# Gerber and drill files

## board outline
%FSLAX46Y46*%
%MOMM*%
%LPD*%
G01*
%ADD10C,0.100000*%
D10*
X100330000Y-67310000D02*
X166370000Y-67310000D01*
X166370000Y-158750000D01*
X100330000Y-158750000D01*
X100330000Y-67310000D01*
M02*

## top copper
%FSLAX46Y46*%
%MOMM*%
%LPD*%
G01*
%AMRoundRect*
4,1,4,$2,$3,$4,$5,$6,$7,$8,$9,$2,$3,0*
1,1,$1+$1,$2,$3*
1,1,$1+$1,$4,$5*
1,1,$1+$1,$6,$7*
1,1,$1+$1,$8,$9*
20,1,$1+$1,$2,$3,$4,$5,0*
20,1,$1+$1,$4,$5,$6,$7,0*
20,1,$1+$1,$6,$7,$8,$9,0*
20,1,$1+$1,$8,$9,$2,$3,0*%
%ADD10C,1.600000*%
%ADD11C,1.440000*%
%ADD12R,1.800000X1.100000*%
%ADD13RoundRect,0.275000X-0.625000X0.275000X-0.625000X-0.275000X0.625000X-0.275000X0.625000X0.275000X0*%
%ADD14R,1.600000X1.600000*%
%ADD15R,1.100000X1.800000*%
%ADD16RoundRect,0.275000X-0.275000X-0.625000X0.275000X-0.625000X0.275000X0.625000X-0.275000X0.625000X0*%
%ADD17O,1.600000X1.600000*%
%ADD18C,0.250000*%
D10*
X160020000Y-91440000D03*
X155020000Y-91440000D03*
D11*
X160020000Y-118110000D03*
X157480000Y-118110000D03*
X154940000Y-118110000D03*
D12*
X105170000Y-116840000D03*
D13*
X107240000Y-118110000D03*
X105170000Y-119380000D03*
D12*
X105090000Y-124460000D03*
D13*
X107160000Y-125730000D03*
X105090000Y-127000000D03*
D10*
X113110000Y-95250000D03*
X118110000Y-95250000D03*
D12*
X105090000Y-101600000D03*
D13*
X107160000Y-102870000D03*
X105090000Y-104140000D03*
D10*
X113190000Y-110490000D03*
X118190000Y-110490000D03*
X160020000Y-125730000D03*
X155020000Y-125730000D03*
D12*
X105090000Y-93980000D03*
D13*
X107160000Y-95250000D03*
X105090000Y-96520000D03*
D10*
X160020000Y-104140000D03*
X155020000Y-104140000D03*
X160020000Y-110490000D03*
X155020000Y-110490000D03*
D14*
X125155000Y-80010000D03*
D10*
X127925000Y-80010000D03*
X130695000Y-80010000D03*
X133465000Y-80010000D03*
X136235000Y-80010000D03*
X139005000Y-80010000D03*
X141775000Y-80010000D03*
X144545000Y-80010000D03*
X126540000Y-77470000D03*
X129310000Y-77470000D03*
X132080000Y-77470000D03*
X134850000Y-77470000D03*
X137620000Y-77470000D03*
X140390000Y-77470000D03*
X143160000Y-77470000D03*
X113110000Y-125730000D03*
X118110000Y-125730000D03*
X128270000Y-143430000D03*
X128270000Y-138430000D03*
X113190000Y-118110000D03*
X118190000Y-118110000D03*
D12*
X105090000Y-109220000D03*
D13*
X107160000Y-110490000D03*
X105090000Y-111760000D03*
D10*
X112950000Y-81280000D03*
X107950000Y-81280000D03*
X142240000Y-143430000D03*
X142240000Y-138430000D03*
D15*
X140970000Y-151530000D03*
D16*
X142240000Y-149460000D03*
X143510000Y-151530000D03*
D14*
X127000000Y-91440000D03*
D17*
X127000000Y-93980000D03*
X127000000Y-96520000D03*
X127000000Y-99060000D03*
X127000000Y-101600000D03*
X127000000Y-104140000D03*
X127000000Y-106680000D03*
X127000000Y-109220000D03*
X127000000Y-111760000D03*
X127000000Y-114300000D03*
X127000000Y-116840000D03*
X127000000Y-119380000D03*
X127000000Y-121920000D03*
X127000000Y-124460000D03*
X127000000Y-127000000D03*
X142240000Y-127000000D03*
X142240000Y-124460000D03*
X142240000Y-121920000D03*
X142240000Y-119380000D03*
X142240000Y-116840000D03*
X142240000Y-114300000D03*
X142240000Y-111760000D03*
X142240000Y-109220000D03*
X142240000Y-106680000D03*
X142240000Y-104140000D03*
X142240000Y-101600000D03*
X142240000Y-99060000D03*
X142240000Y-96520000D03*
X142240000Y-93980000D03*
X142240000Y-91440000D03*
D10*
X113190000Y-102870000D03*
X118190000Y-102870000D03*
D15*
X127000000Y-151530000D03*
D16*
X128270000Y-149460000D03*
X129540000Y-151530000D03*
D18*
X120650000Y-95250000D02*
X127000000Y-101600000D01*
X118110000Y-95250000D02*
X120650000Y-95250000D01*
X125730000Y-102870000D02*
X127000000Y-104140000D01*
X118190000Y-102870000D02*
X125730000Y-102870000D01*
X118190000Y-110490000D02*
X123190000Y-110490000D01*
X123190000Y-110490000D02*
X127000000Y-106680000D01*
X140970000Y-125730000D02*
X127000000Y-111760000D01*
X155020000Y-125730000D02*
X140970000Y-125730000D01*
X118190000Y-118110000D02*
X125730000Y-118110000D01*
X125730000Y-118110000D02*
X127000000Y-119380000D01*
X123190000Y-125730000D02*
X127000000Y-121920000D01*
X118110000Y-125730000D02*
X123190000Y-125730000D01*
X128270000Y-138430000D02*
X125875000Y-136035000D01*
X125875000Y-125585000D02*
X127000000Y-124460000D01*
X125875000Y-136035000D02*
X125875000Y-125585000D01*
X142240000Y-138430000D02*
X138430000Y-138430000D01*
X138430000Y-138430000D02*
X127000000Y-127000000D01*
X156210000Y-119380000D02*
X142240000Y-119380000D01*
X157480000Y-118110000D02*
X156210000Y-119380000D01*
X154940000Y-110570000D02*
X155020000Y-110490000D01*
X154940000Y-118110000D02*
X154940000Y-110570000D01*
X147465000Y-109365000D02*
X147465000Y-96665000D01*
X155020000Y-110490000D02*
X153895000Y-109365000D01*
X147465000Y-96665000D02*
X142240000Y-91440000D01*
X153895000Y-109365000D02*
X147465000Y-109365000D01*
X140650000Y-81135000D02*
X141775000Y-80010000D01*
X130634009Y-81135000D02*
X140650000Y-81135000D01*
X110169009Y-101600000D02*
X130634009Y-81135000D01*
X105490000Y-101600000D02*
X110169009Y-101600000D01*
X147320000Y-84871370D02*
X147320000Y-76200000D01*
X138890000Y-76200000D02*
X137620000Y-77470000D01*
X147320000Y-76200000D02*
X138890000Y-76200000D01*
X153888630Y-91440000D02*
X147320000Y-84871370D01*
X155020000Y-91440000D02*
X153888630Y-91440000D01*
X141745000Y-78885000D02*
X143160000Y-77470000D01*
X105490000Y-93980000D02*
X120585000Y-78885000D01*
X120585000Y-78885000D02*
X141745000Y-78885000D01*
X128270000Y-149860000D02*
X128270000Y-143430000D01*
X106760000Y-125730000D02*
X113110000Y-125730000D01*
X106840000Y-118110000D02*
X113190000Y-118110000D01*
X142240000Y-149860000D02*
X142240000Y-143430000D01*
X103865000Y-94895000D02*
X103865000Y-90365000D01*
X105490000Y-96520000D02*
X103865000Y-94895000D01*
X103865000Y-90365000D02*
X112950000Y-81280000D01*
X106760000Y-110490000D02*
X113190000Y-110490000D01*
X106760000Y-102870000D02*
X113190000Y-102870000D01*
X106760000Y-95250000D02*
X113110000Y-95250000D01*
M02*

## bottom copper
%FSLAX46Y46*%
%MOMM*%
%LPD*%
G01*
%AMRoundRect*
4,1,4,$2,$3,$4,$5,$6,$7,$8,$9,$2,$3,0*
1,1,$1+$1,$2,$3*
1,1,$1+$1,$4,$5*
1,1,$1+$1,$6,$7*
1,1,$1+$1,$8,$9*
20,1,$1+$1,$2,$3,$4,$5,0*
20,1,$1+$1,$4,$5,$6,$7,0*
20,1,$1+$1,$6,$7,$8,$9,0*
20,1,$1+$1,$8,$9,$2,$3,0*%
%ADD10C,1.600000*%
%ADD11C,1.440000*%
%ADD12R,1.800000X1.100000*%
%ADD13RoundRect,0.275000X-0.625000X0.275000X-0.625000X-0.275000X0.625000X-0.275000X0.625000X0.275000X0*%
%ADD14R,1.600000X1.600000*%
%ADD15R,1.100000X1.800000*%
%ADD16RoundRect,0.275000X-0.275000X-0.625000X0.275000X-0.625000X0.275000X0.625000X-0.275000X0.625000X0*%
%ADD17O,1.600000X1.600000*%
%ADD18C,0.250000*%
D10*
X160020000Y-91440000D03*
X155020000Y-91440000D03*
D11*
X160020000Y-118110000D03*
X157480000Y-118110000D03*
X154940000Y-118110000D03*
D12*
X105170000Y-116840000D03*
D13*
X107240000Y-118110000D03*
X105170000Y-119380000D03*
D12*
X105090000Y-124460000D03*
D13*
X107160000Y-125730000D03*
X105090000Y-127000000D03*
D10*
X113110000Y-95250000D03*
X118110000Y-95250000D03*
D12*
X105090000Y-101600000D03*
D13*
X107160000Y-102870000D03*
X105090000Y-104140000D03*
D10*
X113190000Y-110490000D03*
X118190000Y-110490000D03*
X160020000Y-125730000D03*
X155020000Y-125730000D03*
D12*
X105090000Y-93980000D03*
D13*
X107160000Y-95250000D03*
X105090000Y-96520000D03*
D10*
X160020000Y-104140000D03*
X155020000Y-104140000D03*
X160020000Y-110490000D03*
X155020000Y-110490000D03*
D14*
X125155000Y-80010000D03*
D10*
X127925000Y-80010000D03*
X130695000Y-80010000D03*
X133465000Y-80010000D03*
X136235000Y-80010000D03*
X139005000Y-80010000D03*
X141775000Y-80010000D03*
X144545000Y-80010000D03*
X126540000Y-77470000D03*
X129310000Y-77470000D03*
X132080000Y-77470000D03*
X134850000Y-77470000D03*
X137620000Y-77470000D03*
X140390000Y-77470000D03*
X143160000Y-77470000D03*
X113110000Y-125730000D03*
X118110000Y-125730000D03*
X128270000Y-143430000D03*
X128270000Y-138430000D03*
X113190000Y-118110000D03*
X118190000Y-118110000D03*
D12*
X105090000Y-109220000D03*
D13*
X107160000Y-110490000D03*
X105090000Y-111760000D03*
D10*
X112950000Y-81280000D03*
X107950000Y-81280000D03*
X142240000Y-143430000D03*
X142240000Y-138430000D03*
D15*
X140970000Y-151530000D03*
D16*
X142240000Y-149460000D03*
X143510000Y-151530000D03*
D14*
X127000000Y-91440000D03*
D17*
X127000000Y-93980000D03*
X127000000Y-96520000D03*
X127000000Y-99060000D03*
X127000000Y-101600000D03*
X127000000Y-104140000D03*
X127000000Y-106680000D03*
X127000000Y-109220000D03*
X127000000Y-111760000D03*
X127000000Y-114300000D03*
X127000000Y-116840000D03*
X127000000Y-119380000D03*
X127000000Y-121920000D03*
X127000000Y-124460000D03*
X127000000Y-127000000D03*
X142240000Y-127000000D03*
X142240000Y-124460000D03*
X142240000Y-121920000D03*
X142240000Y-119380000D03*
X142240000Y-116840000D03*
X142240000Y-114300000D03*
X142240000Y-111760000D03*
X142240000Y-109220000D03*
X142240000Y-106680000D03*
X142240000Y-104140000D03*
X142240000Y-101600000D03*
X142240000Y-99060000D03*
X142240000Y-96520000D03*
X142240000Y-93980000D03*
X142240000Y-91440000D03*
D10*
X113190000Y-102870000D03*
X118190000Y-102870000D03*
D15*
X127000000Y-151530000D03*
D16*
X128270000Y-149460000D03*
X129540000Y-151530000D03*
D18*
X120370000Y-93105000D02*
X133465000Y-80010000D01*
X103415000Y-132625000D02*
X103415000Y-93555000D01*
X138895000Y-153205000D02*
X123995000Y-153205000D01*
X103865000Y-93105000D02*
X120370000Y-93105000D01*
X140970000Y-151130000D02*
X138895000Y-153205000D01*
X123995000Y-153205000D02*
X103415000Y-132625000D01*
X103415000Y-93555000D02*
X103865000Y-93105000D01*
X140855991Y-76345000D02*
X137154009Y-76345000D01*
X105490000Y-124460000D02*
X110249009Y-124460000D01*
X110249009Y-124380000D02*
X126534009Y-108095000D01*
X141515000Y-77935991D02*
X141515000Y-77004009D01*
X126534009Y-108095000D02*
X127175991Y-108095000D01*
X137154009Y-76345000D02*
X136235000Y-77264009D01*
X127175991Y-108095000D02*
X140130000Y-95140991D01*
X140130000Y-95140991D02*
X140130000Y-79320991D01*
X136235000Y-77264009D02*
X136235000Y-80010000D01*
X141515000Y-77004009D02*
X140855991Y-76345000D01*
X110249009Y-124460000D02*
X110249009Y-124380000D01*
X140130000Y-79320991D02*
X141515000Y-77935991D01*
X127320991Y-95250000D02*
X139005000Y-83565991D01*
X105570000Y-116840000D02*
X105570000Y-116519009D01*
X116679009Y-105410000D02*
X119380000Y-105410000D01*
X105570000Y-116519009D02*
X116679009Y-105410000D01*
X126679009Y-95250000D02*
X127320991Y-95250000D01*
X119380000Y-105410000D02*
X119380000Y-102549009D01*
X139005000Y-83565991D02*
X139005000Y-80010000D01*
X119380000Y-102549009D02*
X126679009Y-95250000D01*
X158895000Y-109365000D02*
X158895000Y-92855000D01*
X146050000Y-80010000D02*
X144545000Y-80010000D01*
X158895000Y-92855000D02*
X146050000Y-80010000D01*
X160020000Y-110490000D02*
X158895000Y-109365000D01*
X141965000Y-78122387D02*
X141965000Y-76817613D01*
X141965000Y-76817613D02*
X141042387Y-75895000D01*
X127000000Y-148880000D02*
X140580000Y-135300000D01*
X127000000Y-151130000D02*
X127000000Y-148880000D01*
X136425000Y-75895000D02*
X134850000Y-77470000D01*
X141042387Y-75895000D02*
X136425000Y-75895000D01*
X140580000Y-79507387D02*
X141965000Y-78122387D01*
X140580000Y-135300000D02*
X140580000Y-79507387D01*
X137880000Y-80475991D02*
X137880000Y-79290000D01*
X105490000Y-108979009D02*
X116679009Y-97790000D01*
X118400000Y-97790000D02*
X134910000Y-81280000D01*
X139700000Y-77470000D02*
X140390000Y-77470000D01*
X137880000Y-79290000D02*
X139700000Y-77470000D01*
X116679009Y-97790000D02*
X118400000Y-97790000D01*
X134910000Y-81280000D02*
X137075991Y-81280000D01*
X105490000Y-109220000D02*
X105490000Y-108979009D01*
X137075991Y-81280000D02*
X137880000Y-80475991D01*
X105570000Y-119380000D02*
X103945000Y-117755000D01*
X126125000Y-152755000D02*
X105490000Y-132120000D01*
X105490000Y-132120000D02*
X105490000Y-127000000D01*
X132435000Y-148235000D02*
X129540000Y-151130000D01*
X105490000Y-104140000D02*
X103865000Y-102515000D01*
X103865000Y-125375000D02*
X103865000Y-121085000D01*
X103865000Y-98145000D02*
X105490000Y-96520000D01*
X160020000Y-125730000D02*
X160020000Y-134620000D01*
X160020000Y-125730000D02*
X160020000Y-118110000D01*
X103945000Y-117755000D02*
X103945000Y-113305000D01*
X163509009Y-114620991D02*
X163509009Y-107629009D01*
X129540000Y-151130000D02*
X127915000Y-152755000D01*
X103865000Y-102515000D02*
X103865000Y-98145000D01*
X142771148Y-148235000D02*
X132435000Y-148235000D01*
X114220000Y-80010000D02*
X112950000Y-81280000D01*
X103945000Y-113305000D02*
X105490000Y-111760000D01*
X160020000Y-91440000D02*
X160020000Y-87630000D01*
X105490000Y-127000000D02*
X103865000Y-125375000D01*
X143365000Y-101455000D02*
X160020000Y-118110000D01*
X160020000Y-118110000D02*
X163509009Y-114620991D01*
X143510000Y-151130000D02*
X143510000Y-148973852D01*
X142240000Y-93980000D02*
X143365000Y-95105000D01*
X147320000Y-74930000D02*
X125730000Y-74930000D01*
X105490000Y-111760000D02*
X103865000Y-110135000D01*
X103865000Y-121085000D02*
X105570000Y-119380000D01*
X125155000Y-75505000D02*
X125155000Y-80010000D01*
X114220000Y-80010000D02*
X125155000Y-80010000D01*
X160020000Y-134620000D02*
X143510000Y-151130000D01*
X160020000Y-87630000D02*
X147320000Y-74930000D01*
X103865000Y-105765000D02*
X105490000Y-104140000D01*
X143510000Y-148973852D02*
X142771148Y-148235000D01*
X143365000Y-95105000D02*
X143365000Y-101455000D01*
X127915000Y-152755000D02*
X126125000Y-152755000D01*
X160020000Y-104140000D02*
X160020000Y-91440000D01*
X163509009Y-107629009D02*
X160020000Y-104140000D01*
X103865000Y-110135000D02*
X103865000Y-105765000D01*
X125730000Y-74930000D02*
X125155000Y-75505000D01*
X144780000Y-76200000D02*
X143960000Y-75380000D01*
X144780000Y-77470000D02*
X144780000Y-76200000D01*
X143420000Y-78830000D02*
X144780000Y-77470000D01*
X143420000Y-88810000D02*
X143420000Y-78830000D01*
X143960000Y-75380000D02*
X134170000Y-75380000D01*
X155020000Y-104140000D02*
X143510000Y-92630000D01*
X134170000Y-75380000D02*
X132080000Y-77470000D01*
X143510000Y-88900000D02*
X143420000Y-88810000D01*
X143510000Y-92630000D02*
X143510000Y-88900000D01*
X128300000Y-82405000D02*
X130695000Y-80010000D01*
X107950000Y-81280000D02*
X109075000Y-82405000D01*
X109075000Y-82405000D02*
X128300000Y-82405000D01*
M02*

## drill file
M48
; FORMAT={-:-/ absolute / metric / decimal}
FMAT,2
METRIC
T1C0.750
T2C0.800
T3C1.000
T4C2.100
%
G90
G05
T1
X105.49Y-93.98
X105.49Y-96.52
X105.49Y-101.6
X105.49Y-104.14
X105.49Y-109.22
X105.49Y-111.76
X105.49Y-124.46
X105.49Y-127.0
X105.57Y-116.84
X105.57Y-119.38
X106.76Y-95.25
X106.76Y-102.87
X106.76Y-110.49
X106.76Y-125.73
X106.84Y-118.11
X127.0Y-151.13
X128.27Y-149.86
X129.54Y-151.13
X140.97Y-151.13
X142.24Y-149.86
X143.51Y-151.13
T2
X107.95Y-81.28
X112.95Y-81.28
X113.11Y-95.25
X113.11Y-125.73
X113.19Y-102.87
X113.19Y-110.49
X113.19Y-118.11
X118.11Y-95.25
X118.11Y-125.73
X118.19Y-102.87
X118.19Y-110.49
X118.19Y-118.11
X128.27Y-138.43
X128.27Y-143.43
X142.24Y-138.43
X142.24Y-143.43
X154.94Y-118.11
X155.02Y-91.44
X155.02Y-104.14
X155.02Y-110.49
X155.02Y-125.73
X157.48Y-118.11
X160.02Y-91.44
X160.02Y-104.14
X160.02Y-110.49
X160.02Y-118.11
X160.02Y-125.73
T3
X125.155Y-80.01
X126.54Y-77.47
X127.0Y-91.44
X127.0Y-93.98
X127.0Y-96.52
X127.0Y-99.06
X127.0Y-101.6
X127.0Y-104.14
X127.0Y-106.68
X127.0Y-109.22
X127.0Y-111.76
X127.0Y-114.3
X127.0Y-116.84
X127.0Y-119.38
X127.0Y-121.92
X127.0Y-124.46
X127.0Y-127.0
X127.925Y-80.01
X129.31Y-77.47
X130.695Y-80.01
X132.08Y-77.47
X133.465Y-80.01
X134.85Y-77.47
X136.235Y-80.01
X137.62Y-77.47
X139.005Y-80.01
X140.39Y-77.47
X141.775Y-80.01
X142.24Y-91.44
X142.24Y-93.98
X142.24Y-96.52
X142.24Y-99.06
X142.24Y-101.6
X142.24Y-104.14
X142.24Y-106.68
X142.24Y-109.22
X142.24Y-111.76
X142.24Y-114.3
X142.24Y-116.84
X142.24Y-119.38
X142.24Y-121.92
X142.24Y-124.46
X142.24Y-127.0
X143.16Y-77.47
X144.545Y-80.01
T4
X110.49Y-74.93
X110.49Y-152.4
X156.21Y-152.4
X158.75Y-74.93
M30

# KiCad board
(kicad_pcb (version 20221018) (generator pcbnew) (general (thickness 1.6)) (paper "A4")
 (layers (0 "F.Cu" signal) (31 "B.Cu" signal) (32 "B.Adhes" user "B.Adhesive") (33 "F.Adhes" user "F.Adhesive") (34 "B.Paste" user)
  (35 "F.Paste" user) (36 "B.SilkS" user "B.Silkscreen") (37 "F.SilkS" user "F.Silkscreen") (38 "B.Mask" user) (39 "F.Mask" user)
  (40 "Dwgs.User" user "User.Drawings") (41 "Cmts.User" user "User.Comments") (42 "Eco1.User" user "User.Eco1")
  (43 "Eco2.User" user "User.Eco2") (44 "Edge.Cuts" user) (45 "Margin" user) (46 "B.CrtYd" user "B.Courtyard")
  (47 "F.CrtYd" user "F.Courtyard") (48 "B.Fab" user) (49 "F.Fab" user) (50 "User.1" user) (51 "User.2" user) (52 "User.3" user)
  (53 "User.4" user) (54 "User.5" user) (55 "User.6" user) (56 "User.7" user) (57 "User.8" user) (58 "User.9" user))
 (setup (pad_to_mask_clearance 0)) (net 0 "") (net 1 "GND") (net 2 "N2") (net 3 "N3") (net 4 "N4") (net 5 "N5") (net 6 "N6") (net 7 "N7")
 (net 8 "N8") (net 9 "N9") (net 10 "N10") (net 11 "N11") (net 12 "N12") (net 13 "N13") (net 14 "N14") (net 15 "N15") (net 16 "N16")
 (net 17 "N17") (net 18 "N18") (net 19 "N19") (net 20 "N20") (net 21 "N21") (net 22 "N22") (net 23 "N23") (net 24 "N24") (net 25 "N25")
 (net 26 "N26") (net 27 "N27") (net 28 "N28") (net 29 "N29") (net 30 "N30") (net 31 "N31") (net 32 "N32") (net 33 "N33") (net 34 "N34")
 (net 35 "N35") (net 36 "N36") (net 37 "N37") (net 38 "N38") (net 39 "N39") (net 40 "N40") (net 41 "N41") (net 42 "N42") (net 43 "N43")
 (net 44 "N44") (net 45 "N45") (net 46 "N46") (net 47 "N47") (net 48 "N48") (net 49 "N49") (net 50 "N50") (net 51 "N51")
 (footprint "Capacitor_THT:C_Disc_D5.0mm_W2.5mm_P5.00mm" (layer "F.Cu") (at 160.02 91.44 180)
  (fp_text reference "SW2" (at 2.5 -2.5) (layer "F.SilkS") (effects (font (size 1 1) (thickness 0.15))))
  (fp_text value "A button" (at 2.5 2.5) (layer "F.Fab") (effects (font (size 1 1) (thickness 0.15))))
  (pad "1" thru_hole circle (at 0 0 180) (size 1.6 1.6) (drill 0.8) (layers "*.Cu" "*.Mask") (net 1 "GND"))
  (pad "2" thru_hole circle (at 5 0 180) (size 1.6 1.6) (drill 0.8) (layers "*.Cu" "*.Mask") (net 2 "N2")))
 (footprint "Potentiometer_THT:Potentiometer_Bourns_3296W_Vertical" (layer "F.Cu") (at 160.02 118.11)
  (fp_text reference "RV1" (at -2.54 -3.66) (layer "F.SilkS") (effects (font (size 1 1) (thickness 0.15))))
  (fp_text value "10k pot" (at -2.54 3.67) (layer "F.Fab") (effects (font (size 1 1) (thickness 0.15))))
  (pad "1" thru_hole circle (at 0 0) (size 1.44 1.44) (drill 0.8) (layers "*.Cu" "*.Mask") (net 1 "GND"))
  (pad "2" thru_hole circle (at -2.54 0) (size 1.44 1.44) (drill 0.8) (layers "*.Cu" "*.Mask") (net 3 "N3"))
  (pad "3" thru_hole circle (at -5.08 0) (size 1.44 1.44) (drill 0.8) (layers "*.Cu" "*.Mask") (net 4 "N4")))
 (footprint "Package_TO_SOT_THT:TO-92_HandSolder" (layer "F.Cu") (at 105.57 116.84 -90)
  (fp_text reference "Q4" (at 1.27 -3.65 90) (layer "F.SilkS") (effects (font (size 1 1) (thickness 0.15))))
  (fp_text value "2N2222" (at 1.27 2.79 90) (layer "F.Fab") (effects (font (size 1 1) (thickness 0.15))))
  (pad "1" thru_hole rect (at 0 0 270) (size 1.1 1.8) (drill 0.75 (offset 0 0.4)) (layers "*.Cu" "*.Mask") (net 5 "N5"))
  (pad "2" thru_hole roundrect (at 1.27 -1.27 270) (size 1.1 1.8) (drill 0.75 (offset 0 -0.4)) (layers "*.Cu" "*.Mask")
   (roundrect_rratio 0.25) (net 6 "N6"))
  (pad "3" thru_hole roundrect (at 2.54 0 270) (size 1.1 1.8) (drill 0.75 (offset 0 0.4)) (layers "*.Cu" "*.Mask") (roundrect_rratio 0.25)
   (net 1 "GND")))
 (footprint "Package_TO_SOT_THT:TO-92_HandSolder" (layer "F.Cu") (at 105.49 124.46 -90)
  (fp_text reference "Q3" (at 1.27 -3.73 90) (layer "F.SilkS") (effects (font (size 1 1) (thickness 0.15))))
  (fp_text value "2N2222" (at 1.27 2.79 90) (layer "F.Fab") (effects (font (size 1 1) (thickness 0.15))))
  (pad "1" thru_hole rect (at 0 0 270) (size 1.1 1.8) (drill 0.75 (offset 0 0.4)) (layers "*.Cu" "*.Mask") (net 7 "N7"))
  (pad "2" thru_hole roundrect (at 1.27 -1.27 270) (size 1.1 1.8) (drill 0.75 (offset 0 -0.4)) (layers "*.Cu" "*.Mask")
   (roundrect_rratio 0.25) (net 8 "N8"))
  (pad "3" thru_hole roundrect (at 2.54 0 270) (size 1.1 1.8) (drill 0.75 (offset 0 0.4)) (layers "*.Cu" "*.Mask") (roundrect_rratio 0.25)
   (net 1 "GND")))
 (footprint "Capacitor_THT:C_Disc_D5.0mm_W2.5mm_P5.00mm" (layer "F.Cu") (at 113.11 95.25)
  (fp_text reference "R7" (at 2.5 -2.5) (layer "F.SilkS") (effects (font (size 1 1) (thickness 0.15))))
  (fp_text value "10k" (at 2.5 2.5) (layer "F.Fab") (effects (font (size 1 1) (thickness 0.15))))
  (pad "1" thru_hole circle (at 0 0) (size 1.6 1.6) (drill 0.8) (layers "*.Cu" "*.Mask") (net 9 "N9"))
  (pad "2" thru_hole circle (at 5 0) (size 1.6 1.6) (drill 0.8) (layers "*.Cu" "*.Mask") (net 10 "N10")))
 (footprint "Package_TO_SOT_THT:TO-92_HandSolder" (layer "F.Cu") (at 105.49 101.6 -90)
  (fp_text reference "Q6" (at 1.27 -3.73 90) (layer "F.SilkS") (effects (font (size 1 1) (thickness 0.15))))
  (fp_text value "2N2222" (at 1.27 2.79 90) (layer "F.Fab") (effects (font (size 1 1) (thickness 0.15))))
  (pad "1" thru_hole rect (at 0 0 270) (size 1.1 1.8) (drill 0.75 (offset 0 0.4)) (layers "*.Cu" "*.Mask") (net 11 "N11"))
  (pad "2" thru_hole roundrect (at 1.27 -1.27 270) (size 1.1 1.8) (drill 0.75 (offset 0 -0.4)) (layers "*.Cu" "*.Mask")
   (roundrect_rratio 0.25) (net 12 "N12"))
  (pad "3" thru_hole roundrect (at 2.54 0 270) (size 1.1 1.8) (drill 0.75 (offset 0 0.4)) (layers "*.Cu" "*.Mask") (roundrect_rratio 0.25)
   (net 1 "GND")))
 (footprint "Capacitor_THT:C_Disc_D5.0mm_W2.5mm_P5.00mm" (layer "F.Cu") (at 113.19 110.49)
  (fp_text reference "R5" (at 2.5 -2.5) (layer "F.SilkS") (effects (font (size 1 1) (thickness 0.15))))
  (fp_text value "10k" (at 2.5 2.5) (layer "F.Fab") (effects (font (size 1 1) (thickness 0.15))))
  (pad "1" thru_hole circle (at 0 0) (size 1.6 1.6) (drill 0.8) (layers "*.Cu" "*.Mask") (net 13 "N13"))
  (pad "2" thru_hole circle (at 5 0) (size 1.6 1.6) (drill 0.8) (layers "*.Cu" "*.Mask") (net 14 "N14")))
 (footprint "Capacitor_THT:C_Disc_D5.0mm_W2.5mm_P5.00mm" (layer "F.Cu") (at 160.02 125.73 180)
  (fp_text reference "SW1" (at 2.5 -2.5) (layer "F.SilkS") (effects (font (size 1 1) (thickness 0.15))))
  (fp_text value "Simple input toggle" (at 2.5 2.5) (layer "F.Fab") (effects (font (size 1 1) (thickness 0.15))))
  (pad "1" thru_hole circle (at 0 0 180) (size 1.6 1.6) (drill 0.8) (layers "*.Cu" "*.Mask") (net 1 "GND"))
  (pad "2" thru_hole circle (at 5 0 180) (size 1.6 1.6) (drill 0.8) (layers "*.Cu" "*.Mask") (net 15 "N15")))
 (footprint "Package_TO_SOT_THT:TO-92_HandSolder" (layer "F.Cu") (at 105.49 93.98 -90)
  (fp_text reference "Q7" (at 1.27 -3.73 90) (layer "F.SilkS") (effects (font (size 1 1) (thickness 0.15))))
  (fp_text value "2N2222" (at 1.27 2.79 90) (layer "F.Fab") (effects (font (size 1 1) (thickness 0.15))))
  (pad "1" thru_hole rect (at 0 0 270) (size 1.1 1.8) (drill 0.75 (offset 0 0.4)) (layers "*.Cu" "*.Mask") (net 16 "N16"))
  (pad "2" thru_hole roundrect (at 1.27 -1.27 270) (size 1.1 1.8) (drill 0.75 (offset 0 -0.4)) (layers "*.Cu" "*.Mask")
   (roundrect_rratio 0.25) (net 9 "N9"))
  (pad "3" thru_hole roundrect (at 2.54 0 270) (size 1.1 1.8) (drill 0.75 (offset 0 0.4)) (layers "*.Cu" "*.Mask") (roundrect_rratio 0.25)
   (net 1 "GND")))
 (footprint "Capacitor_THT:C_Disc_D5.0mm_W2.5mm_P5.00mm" (layer "F.Cu") (at 160.02 104.14 180)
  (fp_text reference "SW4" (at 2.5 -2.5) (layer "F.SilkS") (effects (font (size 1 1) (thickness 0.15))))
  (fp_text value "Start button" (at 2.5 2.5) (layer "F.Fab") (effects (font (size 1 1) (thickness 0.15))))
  (pad "1" thru_hole circle (at 0 0 180) (size 1.6 1.6) (drill 0.8) (layers "*.Cu" "*.Mask") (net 1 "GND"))
  (pad "2" thru_hole circle (at 5 0 180) (size 1.6 1.6) (drill 0.8) (layers "*.Cu" "*.Mask") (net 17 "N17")))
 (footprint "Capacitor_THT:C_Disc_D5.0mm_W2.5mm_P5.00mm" (layer "F.Cu") (at 160.02 110.49 180)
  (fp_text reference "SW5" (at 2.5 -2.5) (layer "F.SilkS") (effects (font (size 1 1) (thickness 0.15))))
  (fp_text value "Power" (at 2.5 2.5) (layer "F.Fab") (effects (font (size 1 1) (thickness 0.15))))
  (pad "1" thru_hole circle (at 0 0 180) (size 1.6 1.6) (drill 0.8) (layers "*.Cu" "*.Mask") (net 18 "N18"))
  (pad "2" thru_hole circle (at 5 0 180) (size 1.6 1.6) (drill 0.8) (layers "*.Cu" "*.Mask") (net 4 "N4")))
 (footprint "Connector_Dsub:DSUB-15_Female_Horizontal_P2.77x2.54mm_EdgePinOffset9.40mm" (layer "F.Cu") (at 125.155 80.01 180)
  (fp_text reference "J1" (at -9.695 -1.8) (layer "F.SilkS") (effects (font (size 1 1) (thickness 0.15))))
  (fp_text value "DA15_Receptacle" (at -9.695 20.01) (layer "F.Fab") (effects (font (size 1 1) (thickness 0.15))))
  (pad "1" thru_hole rect (at 0 0 180) (size 1.6 1.6) (drill 1) (layers "*.Cu" "*.Mask") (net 1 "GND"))
  (pad "2" thru_hole circle (at -2.77 0 180) (size 1.6 1.6) (drill 1) (layers "*.Cu" "*.Mask") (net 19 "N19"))
  (pad "3" thru_hole circle (at -5.54 0 180) (size 1.6 1.6) (drill 1) (layers "*.Cu" "*.Mask") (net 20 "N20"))
  (pad "4" thru_hole circle (at -8.31 0 180) (size 1.6 1.6) (drill 1) (layers "*.Cu" "*.Mask") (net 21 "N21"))
  (pad "5" thru_hole circle (at -11.08 0 180) (size 1.6 1.6) (drill 1) (layers "*.Cu" "*.Mask") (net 7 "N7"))
  (pad "6" thru_hole circle (at -13.85 0 180) (size 1.6 1.6) (drill 1) (layers "*.Cu" "*.Mask") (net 5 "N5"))
  (pad "7" thru_hole circle (at -16.62 0 180) (size 1.6 1.6) (drill 1) (layers "*.Cu" "*.Mask") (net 11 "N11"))
  (pad "8" thru_hole circle (at -19.39 0 180) (size 1.6 1.6) (drill 1) (layers "*.Cu" "*.Mask") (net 18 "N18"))
  (pad "9" thru_hole circle (at -1.385 2.54 180) (size 1.6 1.6) (drill 1) (layers "*.Cu" "*.Mask") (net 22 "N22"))
  (pad "10" thru_hole circle (at -4.155 2.54 180) (size 1.6 1.6) (drill 1) (layers "*.Cu" "*.Mask") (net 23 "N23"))
  (pad "11" thru_hole circle (at -6.925 2.54 180) (size 1.6 1.6) (drill 1) (layers "*.Cu" "*.Mask") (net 17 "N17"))
  (pad "12" thru_hole circle (at -9.695 2.54 180) (size 1.6 1.6) (drill 1) (layers "*.Cu" "*.Mask") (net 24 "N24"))
  (pad "13" thru_hole circle (at -12.465 2.54 180) (size 1.6 1.6) (drill 1) (layers "*.Cu" "*.Mask") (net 2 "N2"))
  (pad "14" thru_hole circle (at -15.235 2.54 180) (size 1.6 1.6) (drill 1) (layers "*.Cu" "*.Mask") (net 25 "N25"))
  (pad "15" thru_hole circle (at -18.005 2.54 180) (size 1.6 1.6) (drill 1) (layers "*.Cu" "*.Mask") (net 16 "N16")))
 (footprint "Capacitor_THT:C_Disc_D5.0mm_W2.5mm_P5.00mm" (layer "F.Cu") (at 113.11 125.73)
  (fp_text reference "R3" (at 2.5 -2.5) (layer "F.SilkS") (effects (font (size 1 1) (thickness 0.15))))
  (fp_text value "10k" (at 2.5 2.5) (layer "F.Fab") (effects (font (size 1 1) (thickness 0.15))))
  (pad "1" thru_hole circle (at 0 0) (size 1.6 1.6) (drill 0.8) (layers "*.Cu" "*.Mask") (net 8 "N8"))
  (pad "2" thru_hole circle (at 5 0) (size 1.6 1.6) (drill 0.8) (layers "*.Cu" "*.Mask") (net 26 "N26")))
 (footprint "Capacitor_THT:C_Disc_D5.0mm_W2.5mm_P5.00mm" (layer "F.Cu") (at 128.27 143.43 90)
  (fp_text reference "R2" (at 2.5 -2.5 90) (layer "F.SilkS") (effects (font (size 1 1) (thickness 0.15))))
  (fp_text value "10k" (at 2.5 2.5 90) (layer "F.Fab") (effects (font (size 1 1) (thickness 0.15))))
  (pad "1" thru_hole circle (at 0 0 90) (size 1.6 1.6) (drill 0.8) (layers "*.Cu" "*.Mask") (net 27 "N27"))
  (pad "2" thru_hole circle (at 5 0 90) (size 1.6 1.6) (drill 0.8) (layers "*.Cu" "*.Mask") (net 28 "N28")))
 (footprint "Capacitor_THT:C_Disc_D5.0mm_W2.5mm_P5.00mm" (layer "F.Cu") (at 113.19 118.11)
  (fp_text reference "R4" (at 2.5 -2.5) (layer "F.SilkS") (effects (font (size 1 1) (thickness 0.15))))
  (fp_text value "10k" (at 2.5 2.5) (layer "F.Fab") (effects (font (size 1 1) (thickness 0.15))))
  (pad "1" thru_hole circle (at 0 0) (size 1.6 1.6) (drill 0.8) (layers "*.Cu" "*.Mask") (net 6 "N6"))
  (pad "2" thru_hole circle (at 5 0) (size 1.6 1.6) (drill 0.8) (layers "*.Cu" "*.Mask") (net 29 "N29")))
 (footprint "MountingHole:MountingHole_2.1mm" (layer "F.Cu") (at 156.21 152.4)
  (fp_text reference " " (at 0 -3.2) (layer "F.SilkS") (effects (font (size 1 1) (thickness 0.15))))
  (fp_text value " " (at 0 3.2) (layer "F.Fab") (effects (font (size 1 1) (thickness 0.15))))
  (pad "" np_thru_hole circle (at 0 0) (size 2.1 2.1) (drill 2.1) (layers "F&B.Cu" "*.Mask")))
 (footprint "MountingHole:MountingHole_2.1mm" (layer "F.Cu") (at 110.49 152.4)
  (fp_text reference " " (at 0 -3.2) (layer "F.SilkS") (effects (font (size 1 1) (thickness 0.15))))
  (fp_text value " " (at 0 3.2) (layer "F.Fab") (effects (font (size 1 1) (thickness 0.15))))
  (pad "" np_thru_hole circle (at 0 0) (size 2.1 2.1) (drill 2.1) (layers "F&B.Cu" "*.Mask")))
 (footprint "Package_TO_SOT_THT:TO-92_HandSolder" (layer "F.Cu") (at 105.49 109.22 -90)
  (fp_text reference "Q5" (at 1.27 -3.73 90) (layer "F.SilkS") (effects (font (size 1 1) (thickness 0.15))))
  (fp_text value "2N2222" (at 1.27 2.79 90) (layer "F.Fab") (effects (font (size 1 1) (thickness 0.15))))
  (pad "1" thru_hole rect (at 0 0 270) (size 1.1 1.8) (drill 0.75 (offset 0 0.4)) (layers "*.Cu" "*.Mask") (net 25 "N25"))
  (pad "2" thru_hole roundrect (at 1.27 -1.27 270) (size 1.1 1.8) (drill 0.75 (offset 0 -0.4)) (layers "*.Cu" "*.Mask")
   (roundrect_rratio 0.25) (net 13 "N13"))
  (pad "3" thru_hole roundrect (at 2.54 0 270) (size 1.1 1.8) (drill 0.75 (offset 0 0.4)) (layers "*.Cu" "*.Mask") (roundrect_rratio 0.25)
   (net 1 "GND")))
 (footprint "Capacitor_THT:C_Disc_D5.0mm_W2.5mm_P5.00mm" (layer "F.Cu") (at 112.95 81.28 180)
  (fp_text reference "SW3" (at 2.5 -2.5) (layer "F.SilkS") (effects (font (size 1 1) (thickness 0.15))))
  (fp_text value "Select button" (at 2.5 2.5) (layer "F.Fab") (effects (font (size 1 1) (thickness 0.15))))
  (pad "1" thru_hole circle (at 0 0 180) (size 1.6 1.6) (drill 0.8) (layers "*.Cu" "*.Mask") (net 1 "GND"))
  (pad "2" thru_hole circle (at 5 0 180) (size 1.6 1.6) (drill 0.8) (layers "*.Cu" "*.Mask") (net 20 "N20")))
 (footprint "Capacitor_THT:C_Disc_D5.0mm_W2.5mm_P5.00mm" (layer "F.Cu") (at 142.24 143.43 90)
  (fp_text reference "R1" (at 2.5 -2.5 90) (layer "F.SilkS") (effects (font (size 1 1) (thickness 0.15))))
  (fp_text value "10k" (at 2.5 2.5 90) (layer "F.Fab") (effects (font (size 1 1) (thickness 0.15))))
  (pad "1" thru_hole circle (at 0 0 90) (size 1.6 1.6) (drill 0.8) (layers "*.Cu" "*.Mask") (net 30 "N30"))
  (pad "2" thru_hole circle (at 5 0 90) (size 1.6 1.6) (drill 0.8) (layers "*.Cu" "*.Mask") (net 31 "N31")))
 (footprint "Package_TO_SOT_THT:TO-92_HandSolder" (layer "F.Cu") (at 140.97 151.13)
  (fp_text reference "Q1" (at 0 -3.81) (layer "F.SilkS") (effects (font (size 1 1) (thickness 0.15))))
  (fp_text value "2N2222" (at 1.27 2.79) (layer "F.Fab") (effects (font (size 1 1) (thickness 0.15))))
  (pad "1" thru_hole rect (at 0 0) (size 1.1 1.8) (drill 0.75 (offset 0 0.4)) (layers "*.Cu" "*.Mask") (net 21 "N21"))
  (pad "2" thru_hole roundrect (at 1.27 -1.27) (size 1.1 1.8) (drill 0.75 (offset 0 -0.4)) (layers "*.Cu" "*.Mask") (roundrect_rratio 0.25)
   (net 30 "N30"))
  (pad "3" thru_hole roundrect (at 2.54 0) (size 1.1 1.8) (drill 0.75 (offset 0 0.4)) (layers "*.Cu" "*.Mask") (roundrect_rratio 0.25)
   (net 1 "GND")))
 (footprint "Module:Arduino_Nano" (layer "F.Cu") (at 127 91.44)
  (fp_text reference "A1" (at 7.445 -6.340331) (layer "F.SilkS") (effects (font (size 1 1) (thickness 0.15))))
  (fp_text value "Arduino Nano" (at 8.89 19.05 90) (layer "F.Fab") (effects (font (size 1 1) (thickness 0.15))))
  (pad "1" thru_hole rect (at 0 0) (size 1.6 1.6) (drill 1) (layers "*.Cu" "*.Mask") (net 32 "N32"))
  (pad "2" thru_hole oval (at 0 2.54) (size 1.6 1.6) (drill 1) (layers "*.Cu" "*.Mask") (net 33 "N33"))
  (pad "3" thru_hole oval (at 0 5.08) (size 1.6 1.6) (drill 1) (layers "*.Cu" "*.Mask") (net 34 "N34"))
  (pad "4" thru_hole oval (at 0 7.62) (size 1.6 1.6) (drill 1) (layers "*.Cu" "*.Mask") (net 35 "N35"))
  (pad "5" thru_hole oval (at 0 10.16) (size 1.6 1.6) (drill 1) (layers "*.Cu" "*.Mask") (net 10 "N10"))
  (pad "6" thru_hole oval (at 0 12.7) (size 1.6 1.6) (drill 1) (layers "*.Cu" "*.Mask") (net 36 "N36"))
  (pad "7" thru_hole oval (at 0 15.24) (size 1.6 1.6) (drill 1) (layers "*.Cu" "*.Mask") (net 14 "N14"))
  (pad "8" thru_hole oval (at 0 17.78) (size 1.6 1.6) (drill 1) (layers "*.Cu" "*.Mask") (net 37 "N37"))
  (pad "9" thru_hole oval (at 0 20.32) (size 1.6 1.6) (drill 1) (layers "*.Cu" "*.Mask") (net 15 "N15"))
  (pad "10" thru_hole oval (at 0 22.86) (size 1.6 1.6) (drill 1) (layers "*.Cu" "*.Mask") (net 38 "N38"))
  (pad "11" thru_hole oval (at 0 25.4) (size 1.6 1.6) (drill 1) (layers "*.Cu" "*.Mask") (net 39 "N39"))
  (pad "12" thru_hole oval (at 0 27.94) (size 1.6 1.6) (drill 1) (layers "*.Cu" "*.Mask") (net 29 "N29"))
  (pad "13" thru_hole oval (at 0 30.48) (size 1.6 1.6) (drill 1) (layers "*.Cu" "*.Mask") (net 26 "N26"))
  (pad "14" thru_hole oval (at 0 33.02) (size 1.6 1.6) (drill 1) (layers "*.Cu" "*.Mask") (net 28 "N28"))
  (pad "15" thru_hole oval (at 0 35.56) (size 1.6 1.6) (drill 1) (layers "*.Cu" "*.Mask") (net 31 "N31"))
  (pad "16" thru_hole oval (at 15.24 35.56) (size 1.6 1.6) (drill 1) (layers "*.Cu" "*.Mask") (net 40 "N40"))
  (pad "17" thru_hole oval (at 15.24 33.02) (size 1.6 1.6) (drill 1) (layers "*.Cu" "*.Mask") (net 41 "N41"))
  (pad "18" thru_hole oval (at 15.24 30.48) (size 1.6 1.6) (drill 1) (layers "*.Cu" "*.Mask") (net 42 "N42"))
  (pad "19" thru_hole oval (at 15.24 27.94) (size 1.6 1.6) (drill 1) (layers "*.Cu" "*.Mask") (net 3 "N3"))
  (pad "20" thru_hole oval (at 15.24 25.4) (size 1.6 1.6) (drill 1) (layers "*.Cu" "*.Mask") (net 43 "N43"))
  (pad "21" thru_hole oval (at 15.24 22.86) (size 1.6 1.6) (drill 1) (layers "*.Cu" "*.Mask") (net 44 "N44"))
  (pad "22" thru_hole oval (at 15.24 20.32) (size 1.6 1.6) (drill 1) (layers "*.Cu" "*.Mask") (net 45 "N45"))
  (pad "23" thru_hole oval (at 15.24 17.78) (size 1.6 1.6) (drill 1) (layers "*.Cu" "*.Mask") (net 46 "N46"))
  (pad "24" thru_hole oval (at 15.24 15.24) (size 1.6 1.6) (drill 1) (layers "*.Cu" "*.Mask") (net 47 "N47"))
  (pad "25" thru_hole oval (at 15.24 12.7) (size 1.6 1.6) (drill 1) (layers "*.Cu" "*.Mask") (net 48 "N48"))
  (pad "26" thru_hole oval (at 15.24 10.16) (size 1.6 1.6) (drill 1) (layers "*.Cu" "*.Mask") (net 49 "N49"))
  (pad "27" thru_hole oval (at 15.24 7.62) (size 1.6 1.6) (drill 1) (layers "*.Cu" "*.Mask") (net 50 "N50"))
  (pad "28" thru_hole oval (at 15.24 5.08) (size 1.6 1.6) (drill 1) (layers "*.Cu" "*.Mask") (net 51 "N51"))
  (pad "29" thru_hole oval (at 15.24 2.54) (size 1.6 1.6) (drill 1) (layers "*.Cu" "*.Mask") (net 1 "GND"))
  (pad "30" thru_hole oval (at 15.24 0) (size 1.6 1.6) (drill 1) (layers "*.Cu" "*.Mask") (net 4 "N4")))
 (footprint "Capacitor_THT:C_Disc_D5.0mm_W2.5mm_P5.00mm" (layer "F.Cu") (at 113.19 102.87)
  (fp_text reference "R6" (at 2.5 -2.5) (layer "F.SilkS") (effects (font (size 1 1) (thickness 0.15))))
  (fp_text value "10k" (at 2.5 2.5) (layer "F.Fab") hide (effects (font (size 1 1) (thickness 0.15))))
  (pad "1" thru_hole circle (at 0 0) (size 1.6 1.6) (drill 0.8) (layers "*.Cu" "*.Mask") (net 12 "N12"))
  (pad "2" thru_hole circle (at 5 0) (size 1.6 1.6) (drill 0.8) (layers "*.Cu" "*.Mask") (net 36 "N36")))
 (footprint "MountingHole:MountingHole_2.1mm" (layer "F.Cu") (at 110.49 74.93)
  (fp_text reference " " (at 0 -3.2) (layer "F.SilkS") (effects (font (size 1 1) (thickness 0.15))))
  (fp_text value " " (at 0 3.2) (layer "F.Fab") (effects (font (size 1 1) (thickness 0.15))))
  (pad "" np_thru_hole circle (at 0 0) (size 2.1 2.1) (drill 2.1) (layers "*.Cu" "*.Mask")))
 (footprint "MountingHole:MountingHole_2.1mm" (layer "F.Cu") (at 158.75 74.93)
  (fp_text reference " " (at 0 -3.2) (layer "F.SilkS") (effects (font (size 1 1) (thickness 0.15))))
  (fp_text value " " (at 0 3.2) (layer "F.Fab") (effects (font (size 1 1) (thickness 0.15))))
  (pad "" np_thru_hole circle (at 0 0) (size 2.1 2.1) (drill 2.1) (layers "F&B.Cu" "*.Mask")))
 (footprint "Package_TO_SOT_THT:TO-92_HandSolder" (layer "F.Cu") (at 127 151.13)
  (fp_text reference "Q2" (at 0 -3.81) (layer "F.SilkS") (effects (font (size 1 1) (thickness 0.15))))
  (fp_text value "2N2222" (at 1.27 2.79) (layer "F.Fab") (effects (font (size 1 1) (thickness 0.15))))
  (pad "1" thru_hole rect (at 0 0) (size 1.1 1.8) (drill 0.75 (offset 0 0.4)) (layers "*.Cu" "*.Mask") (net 24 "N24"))
  (pad "2" thru_hole roundrect (at 1.27 -1.27) (size 1.1 1.8) (drill 0.75 (offset 0 -0.4)) (layers "*.Cu" "*.Mask") (roundrect_rratio 0.25)
   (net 27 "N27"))
  (pad "3" thru_hole roundrect (at 2.54 0) (size 1.1 1.8) (drill 0.75 (offset 0 0.4)) (layers "*.Cu" "*.Mask") (roundrect_rratio 0.25)
   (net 1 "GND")))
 (gr_rect (start 100.33 67.31) (end 166.37 158.75) (stroke (width 0.1) (type default)) (fill none) (layer "Edge.Cuts"))
 (segment (start 120.65 95.25) (end 127 101.6) (width 0.25) (layer "F.Cu") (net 10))
 (segment (start 118.11 95.25) (end 120.65 95.25) (width 0.25) (layer "F.Cu") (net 10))
 (segment (start 125.73 102.87) (end 127 104.14) (width 0.25) (layer "F.Cu") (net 36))
 (segment (start 118.19 102.87) (end 125.73 102.87) (width 0.25) (layer "F.Cu") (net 36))
 (segment (start 118.19 110.49) (end 123.19 110.49) (width 0.25) (layer "F.Cu") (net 14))
 (segment (start 123.19 110.49) (end 127 106.68) (width 0.25) (layer "F.Cu") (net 14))
 (segment (start 140.97 125.73) (end 127 111.76) (width 0.25) (layer "F.Cu") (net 15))
 (segment (start 155.02 125.73) (end 140.97 125.73) (width 0.25) (layer "F.Cu") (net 15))
 (segment (start 118.19 118.11) (end 125.73 118.11) (width 0.25) (layer "F.Cu") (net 29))
 (segment (start 125.73 118.11) (end 127 119.38) (width 0.25) (layer "F.Cu") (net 29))
 (segment (start 123.19 125.73) (end 127 121.92) (width 0.25) (layer "F.Cu") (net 26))
 (segment (start 118.11 125.73) (end 123.19 125.73) (width 0.25) (layer "F.Cu") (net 26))
 (segment (start 128.27 138.43) (end 125.875 136.035) (width 0.25) (layer "F.Cu") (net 28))
 (segment (start 125.875 125.585) (end 127 124.46) (width 0.25) (layer "F.Cu") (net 28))
 (segment (start 125.875 136.035) (end 125.875 125.585) (width 0.25) (layer "F.Cu") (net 28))
 (segment (start 142.24 138.43) (end 138.43 138.43) (width 0.25) (layer "F.Cu") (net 31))
 (segment (start 138.43 138.43) (end 127 127) (width 0.25) (layer "F.Cu") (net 31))
 (segment (start 156.21 119.38) (end 142.24 119.38) (width 0.25) (layer "F.Cu") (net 3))
 (segment (start 157.48 118.11) (end 156.21 119.38) (width 0.25) (layer "F.Cu") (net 3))
 (segment (start 154.94 110.57) (end 155.02 110.49) (width 0.25) (layer "F.Cu") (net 4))
 (segment (start 154.94 118.11) (end 154.94 110.57) (width 0.25) (layer "F.Cu") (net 4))
 (segment (start 147.465 109.365) (end 147.465 96.665) (width 0.25) (layer "F.Cu") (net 4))
 (segment (start 155.02 110.49) (end 153.895 109.365) (width 0.25) (layer "F.Cu") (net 4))
 (segment (start 147.465 96.665) (end 142.24 91.44) (width 0.25) (layer "F.Cu") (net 4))
 (segment (start 153.895 109.365) (end 147.465 109.365) (width 0.25) (layer "F.Cu") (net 4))
 (segment (start 120.37 93.105) (end 133.465 80.01) (width 0.25) (layer "B.Cu") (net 21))
 (segment (start 103.415 132.625) (end 103.415 93.555) (width 0.25) (layer "B.Cu") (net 21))
 (segment (start 138.895 153.205) (end 123.995 153.205) (width 0.25) (layer "B.Cu") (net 21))
 (segment (start 103.865 93.105) (end 120.37 93.105) (width 0.25) (layer "B.Cu") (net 21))
 (segment (start 140.97 151.13) (end 138.895 153.205) (width 0.25) (layer "B.Cu") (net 21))
 (segment (start 123.995 153.205) (end 103.415 132.625) (width 0.25) (layer "B.Cu") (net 21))
 (segment (start 103.415 93.555) (end 103.865 93.105) (width 0.25) (layer "B.Cu") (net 21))
 (segment (start 140.855991 76.345) (end 137.154009 76.345) (width 0.25) (layer "B.Cu") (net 7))
 (segment (start 105.49 124.46) (end 110.249009 124.46) (width 0.25) (layer "B.Cu") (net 7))
 (segment (start 110.249009 124.38) (end 126.534009 108.095) (width 0.25) (layer "B.Cu") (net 7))
 (segment (start 141.515 77.935991) (end 141.515 77.004009) (width 0.25) (layer "B.Cu") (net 7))
 (segment (start 126.534009 108.095) (end 127.175991 108.095) (width 0.25) (layer "B.Cu") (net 7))
 (segment (start 137.154009 76.345) (end 136.235 77.264009) (width 0.25) (layer "B.Cu") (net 7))
 (segment (start 127.175991 108.095) (end 140.13 95.140991) (width 0.25) (layer "B.Cu") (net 7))
 (segment (start 140.13 95.140991) (end 140.13 79.320991) (width 0.25) (layer "B.Cu") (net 7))
 (segment (start 136.235 77.264009) (end 136.235 80.01) (width 0.25) (layer "B.Cu") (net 7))
 (segment (start 141.515 77.004009) (end 140.855991 76.345) (width 0.25) (layer "B.Cu") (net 7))
 (segment (start 110.249009 124.46) (end 110.249009 124.38) (width 0.25) (layer "B.Cu") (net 7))
 (segment (start 140.13 79.320991) (end 141.515 77.935991) (width 0.25) (layer "B.Cu") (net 7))
 (segment (start 127.320991 95.25) (end 139.005 83.565991) (width 0.25) (layer "B.Cu") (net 5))
 (segment (start 105.57 116.84) (end 105.57 116.519009) (width 0.25) (layer "B.Cu") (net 5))
 (segment (start 116.679009 105.41) (end 119.38 105.41) (width 0.25) (layer "B.Cu") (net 5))
 (segment (start 105.57 116.519009) (end 116.679009 105.41) (width 0.25) (layer "B.Cu") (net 5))
 (segment (start 126.679009 95.25) (end 127.320991 95.25) (width 0.25) (layer "B.Cu") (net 5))
 (segment (start 119.38 105.41) (end 119.38 102.549009) (width 0.25) (layer "B.Cu") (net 5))
 (segment (start 139.005 83.565991) (end 139.005 80.01) (width 0.25) (layer "B.Cu") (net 5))
 (segment (start 119.38 102.549009) (end 126.679009 95.25) (width 0.25) (layer "B.Cu") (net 5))
 (segment (start 140.65 81.135) (end 141.775 80.01) (width 0.25) (layer "F.Cu") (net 11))
 (segment (start 130.634009 81.135) (end 140.65 81.135) (width 0.25) (layer "F.Cu") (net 11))
 (segment (start 110.169009 101.6) (end 130.634009 81.135) (width 0.25) (layer "F.Cu") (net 11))
 (segment (start 105.49 101.6) (end 110.169009 101.6) (width 0.25) (layer "F.Cu") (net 11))
 (segment (start 158.895 109.365) (end 158.895 92.855) (width 0.25) (layer "B.Cu") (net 18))
 (segment (start 146.05 80.01) (end 144.545 80.01) (width 0.25) (layer "B.Cu") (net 18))
 (segment (start 158.895 92.855) (end 146.05 80.01) (width 0.25) (layer "B.Cu") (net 18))
 (segment (start 160.02 110.49) (end 158.895 109.365) (width 0.25) (layer "B.Cu") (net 18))
 (segment (start 141.965 78.122387) (end 141.965 76.817613) (width 0.25) (layer "B.Cu") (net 24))
 (segment (start 141.965 76.817613) (end 141.042387 75.895) (width 0.25) (layer "B.Cu") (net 24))
 (segment (start 127 148.88) (end 140.58 135.3) (width 0.25) (layer "B.Cu") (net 24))
 (segment (start 127 151.13) (end 127 148.88) (width 0.25) (layer "B.Cu") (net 24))
 (segment (start 136.425 75.895) (end 134.85 77.47) (width 0.25) (layer "B.Cu") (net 24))
 (segment (start 141.042387 75.895) (end 136.425 75.895) (width 0.25) (layer "B.Cu") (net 24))
 (segment (start 140.58 79.507387) (end 141.965 78.122387) (width 0.25) (layer "B.Cu") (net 24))
 (segment (start 140.58 135.3) (end 140.58 79.507387) (width 0.25) (layer "B.Cu") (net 24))
 (segment (start 147.32 84.87137) (end 147.32 76.2) (width 0.25) (layer "F.Cu") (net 2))
 (segment (start 138.89 76.2) (end 137.62 77.47) (width 0.25) (layer "F.Cu") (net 2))
 (segment (start 147.32 76.2) (end 138.89 76.2) (width 0.25) (layer "F.Cu") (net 2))
 (segment (start 153.88863 91.44) (end 147.32 84.87137) (width 0.25) (layer "F.Cu") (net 2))
 (segment (start 155.02 91.44) (end 153.88863 91.44) (width 0.25) (layer "F.Cu") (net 2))
 (segment (start 137.88 80.475991) (end 137.88 79.29) (width 0.25) (layer "B.Cu") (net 25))
 (segment (start 105.49 108.979009) (end 116.679009 97.79) (width 0.25) (layer "B.Cu") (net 25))
 (segment (start 118.4 97.79) (end 134.91 81.28) (width 0.25) (layer "B.Cu") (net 25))
 (segment (start 139.7 77.47) (end 140.39 77.47) (width 0.25) (layer "B.Cu") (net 25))
 (segment (start 137.88 79.29) (end 139.7 77.47) (width 0.25) (layer "B.Cu") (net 25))
 (segment (start 116.679009 97.79) (end 118.4 97.79) (width 0.25) (layer "B.Cu") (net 25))
 (segment (start 134.91 81.28) (end 137.075991 81.28) (width 0.25) (layer "B.Cu") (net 25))
 (segment (start 105.49 109.22) (end 105.49 108.979009) (width 0.25) (layer "B.Cu") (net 25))
 (segment (start 137.075991 81.28) (end 137.88 80.475991) (width 0.25) (layer "B.Cu") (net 25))
 (segment (start 141.745 78.885) (end 143.16 77.47) (width 0.25) (layer "F.Cu") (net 16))
 (segment (start 105.49 93.98) (end 120.585 78.885) (width 0.25) (layer "F.Cu") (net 16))
 (segment (start 120.585 78.885) (end 141.745 78.885) (width 0.25) (layer "F.Cu") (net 16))
 (segment (start 128.27 149.86) (end 128.27 143.43) (width 0.25) (layer "F.Cu") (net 27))
 (segment (start 106.76 125.73) (end 113.11 125.73) (width 0.25) (layer "F.Cu") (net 8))
 (segment (start 106.84 118.11) (end 113.19 118.11) (width 0.25) (layer "F.Cu") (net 6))
 (segment (start 142.24 149.86) (end 142.24 143.43) (width 0.25) (layer "F.Cu") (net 30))
 (segment (start 103.865 94.895) (end 103.865 90.365) (width 0.25) (layer "F.Cu") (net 1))
 (segment (start 105.49 96.52) (end 103.865 94.895) (width 0.25) (layer "F.Cu") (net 1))
 (segment (start 103.865 90.365) (end 112.95 81.28) (width 0.25) (layer "F.Cu") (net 1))
 (segment (start 105.57 119.38) (end 103.945 117.755) (width 0.25) (layer "B.Cu") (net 1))
 (segment (start 126.125 152.755) (end 105.49 132.12) (width 0.25) (layer "B.Cu") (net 1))
 (segment (start 105.49 132.12) (end 105.49 127) (width 0.25) (layer "B.Cu") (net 1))
 (segment (start 132.435 148.235) (end 129.54 151.13) (width 0.25) (layer "B.Cu") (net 1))
 (segment (start 105.49 104.14) (end 103.865 102.515) (width 0.25) (layer "B.Cu") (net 1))
 (segment (start 103.865 125.375) (end 103.865 121.085) (width 0.25) (layer "B.Cu") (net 1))
 (segment (start 103.865 98.145) (end 105.49 96.52) (width 0.25) (layer "B.Cu") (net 1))
 (segment (start 160.02 125.73) (end 160.02 134.62) (width 0.25) (layer "B.Cu") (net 1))
 (segment (start 160.02 125.73) (end 160.02 118.11) (width 0.25) (layer "B.Cu") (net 1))
 (segment (start 103.945 117.755) (end 103.945 113.305) (width 0.25) (layer "B.Cu") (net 1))
 (segment (start 163.509009 114.620991) (end 163.509009 107.629009) (width 0.25) (layer "B.Cu") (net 1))
 (segment (start 129.54 151.13) (end 127.915 152.755) (width 0.25) (layer "B.Cu") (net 1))
 (segment (start 103.865 102.515) (end 103.865 98.145) (width 0.25) (layer "B.Cu") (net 1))
 (segment (start 142.771148 148.235) (end 132.435 148.235) (width 0.25) (layer "B.Cu") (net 1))
 (segment (start 114.22 80.01) (end 112.95 81.28) (width 0.25) (layer "B.Cu") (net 1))
 (segment (start 103.945 113.305) (end 105.49 111.76) (width 0.25) (layer "B.Cu") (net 1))
 (segment (start 160.02 91.44) (end 160.02 87.63) (width 0.25) (layer "B.Cu") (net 1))
 (segment (start 105.49 127) (end 103.865 125.375) (width 0.25) (layer "B.Cu") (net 1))
 (segment (start 143.365 101.455) (end 160.02 118.11) (width 0.25) (layer "B.Cu") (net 1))
 (segment (start 160.02 118.11) (end 163.509009 114.620991) (width 0.25) (layer "B.Cu") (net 1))
 (segment (start 143.51 151.13) (end 143.51 148.973852) (width 0.25) (layer "B.Cu") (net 1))
 (segment (start 142.24 93.98) (end 143.365 95.105) (width 0.25) (layer "B.Cu") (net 1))
 (segment (start 147.32 74.93) (end 125.73 74.93) (width 0.25) (layer "B.Cu") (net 1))
 (segment (start 105.49 111.76) (end 103.865 110.135) (width 0.25) (layer "B.Cu") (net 1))
 (segment (start 103.865 121.085) (end 105.57 119.38) (width 0.25) (layer "B.Cu") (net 1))
 (segment (start 125.155 75.505) (end 125.155 80.01) (width 0.25) (layer "B.Cu") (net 1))
 (segment (start 114.22 80.01) (end 125.155 80.01) (width 0.25) (layer "B.Cu") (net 1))
 (segment (start 160.02 134.62) (end 143.51 151.13) (width 0.25) (layer "B.Cu") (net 1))
 (segment (start 160.02 87.63) (end 147.32 74.93) (width 0.25) (layer "B.Cu") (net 1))
 (segment (start 103.865 105.765) (end 105.49 104.14) (width 0.25) (layer "B.Cu") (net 1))
 (segment (start 143.51 148.973852) (end 142.771148 148.235) (width 0.25) (layer "B.Cu") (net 1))
 (segment (start 143.365 95.105) (end 143.365 101.455) (width 0.25) (layer "B.Cu") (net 1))
 (segment (start 127.915 152.755) (end 126.125 152.755) (width 0.25) (layer "B.Cu") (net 1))
 (segment (start 160.02 104.14) (end 160.02 91.44) (width 0.25) (layer "B.Cu") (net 1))
 (segment (start 163.509009 107.629009) (end 160.02 104.14) (width 0.25) (layer "B.Cu") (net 1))
 (segment (start 103.865 110.135) (end 103.865 105.765) (width 0.25) (layer "B.Cu") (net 1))
 (segment (start 125.73 74.93) (end 125.155 75.505) (width 0.25) (layer "B.Cu") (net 1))
 (segment (start 106.76 110.49) (end 113.19 110.49) (width 0.25) (layer "F.Cu") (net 13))
 (segment (start 106.76 102.87) (end 113.19 102.87) (width 0.25) (layer "F.Cu") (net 12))
 (segment (start 106.76 95.25) (end 113.11 95.25) (width 0.25) (layer "F.Cu") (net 9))
 (segment (start 144.78 76.2) (end 143.96 75.38) (width 0.25) (layer "B.Cu") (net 17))
 (segment (start 144.78 77.47) (end 144.78 76.2) (width 0.25) (layer "B.Cu") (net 17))
 (segment (start 143.42 78.83) (end 144.78 77.47) (width 0.25) (layer "B.Cu") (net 17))
 (segment (start 143.42 88.81) (end 143.42 78.83) (width 0.25) (layer "B.Cu") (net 17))
 (segment (start 143.96 75.38) (end 134.17 75.38) (width 0.25) (layer "B.Cu") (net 17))
 (segment (start 155.02 104.14) (end 143.51 92.63) (width 0.25) (layer "B.Cu") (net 17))
 (segment (start 134.17 75.38) (end 132.08 77.47) (width 0.25) (layer "B.Cu") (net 17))
 (segment (start 143.51 88.9) (end 143.42 88.81) (width 0.25) (layer "B.Cu") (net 17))
 (segment (start 143.51 92.63) (end 143.51 88.9) (width 0.25) (layer "B.Cu") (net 17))
 (segment (start 128.3 82.405) (end 130.695 80.01) (width 0.25) (layer "B.Cu") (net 20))
 (segment (start 107.95 81.28) (end 109.075 82.405) (width 0.25) (layer "B.Cu") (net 20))
 (segment (start 109.075 82.405) (end 128.3 82.405) (width 0.25) (layer "B.Cu") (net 20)))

